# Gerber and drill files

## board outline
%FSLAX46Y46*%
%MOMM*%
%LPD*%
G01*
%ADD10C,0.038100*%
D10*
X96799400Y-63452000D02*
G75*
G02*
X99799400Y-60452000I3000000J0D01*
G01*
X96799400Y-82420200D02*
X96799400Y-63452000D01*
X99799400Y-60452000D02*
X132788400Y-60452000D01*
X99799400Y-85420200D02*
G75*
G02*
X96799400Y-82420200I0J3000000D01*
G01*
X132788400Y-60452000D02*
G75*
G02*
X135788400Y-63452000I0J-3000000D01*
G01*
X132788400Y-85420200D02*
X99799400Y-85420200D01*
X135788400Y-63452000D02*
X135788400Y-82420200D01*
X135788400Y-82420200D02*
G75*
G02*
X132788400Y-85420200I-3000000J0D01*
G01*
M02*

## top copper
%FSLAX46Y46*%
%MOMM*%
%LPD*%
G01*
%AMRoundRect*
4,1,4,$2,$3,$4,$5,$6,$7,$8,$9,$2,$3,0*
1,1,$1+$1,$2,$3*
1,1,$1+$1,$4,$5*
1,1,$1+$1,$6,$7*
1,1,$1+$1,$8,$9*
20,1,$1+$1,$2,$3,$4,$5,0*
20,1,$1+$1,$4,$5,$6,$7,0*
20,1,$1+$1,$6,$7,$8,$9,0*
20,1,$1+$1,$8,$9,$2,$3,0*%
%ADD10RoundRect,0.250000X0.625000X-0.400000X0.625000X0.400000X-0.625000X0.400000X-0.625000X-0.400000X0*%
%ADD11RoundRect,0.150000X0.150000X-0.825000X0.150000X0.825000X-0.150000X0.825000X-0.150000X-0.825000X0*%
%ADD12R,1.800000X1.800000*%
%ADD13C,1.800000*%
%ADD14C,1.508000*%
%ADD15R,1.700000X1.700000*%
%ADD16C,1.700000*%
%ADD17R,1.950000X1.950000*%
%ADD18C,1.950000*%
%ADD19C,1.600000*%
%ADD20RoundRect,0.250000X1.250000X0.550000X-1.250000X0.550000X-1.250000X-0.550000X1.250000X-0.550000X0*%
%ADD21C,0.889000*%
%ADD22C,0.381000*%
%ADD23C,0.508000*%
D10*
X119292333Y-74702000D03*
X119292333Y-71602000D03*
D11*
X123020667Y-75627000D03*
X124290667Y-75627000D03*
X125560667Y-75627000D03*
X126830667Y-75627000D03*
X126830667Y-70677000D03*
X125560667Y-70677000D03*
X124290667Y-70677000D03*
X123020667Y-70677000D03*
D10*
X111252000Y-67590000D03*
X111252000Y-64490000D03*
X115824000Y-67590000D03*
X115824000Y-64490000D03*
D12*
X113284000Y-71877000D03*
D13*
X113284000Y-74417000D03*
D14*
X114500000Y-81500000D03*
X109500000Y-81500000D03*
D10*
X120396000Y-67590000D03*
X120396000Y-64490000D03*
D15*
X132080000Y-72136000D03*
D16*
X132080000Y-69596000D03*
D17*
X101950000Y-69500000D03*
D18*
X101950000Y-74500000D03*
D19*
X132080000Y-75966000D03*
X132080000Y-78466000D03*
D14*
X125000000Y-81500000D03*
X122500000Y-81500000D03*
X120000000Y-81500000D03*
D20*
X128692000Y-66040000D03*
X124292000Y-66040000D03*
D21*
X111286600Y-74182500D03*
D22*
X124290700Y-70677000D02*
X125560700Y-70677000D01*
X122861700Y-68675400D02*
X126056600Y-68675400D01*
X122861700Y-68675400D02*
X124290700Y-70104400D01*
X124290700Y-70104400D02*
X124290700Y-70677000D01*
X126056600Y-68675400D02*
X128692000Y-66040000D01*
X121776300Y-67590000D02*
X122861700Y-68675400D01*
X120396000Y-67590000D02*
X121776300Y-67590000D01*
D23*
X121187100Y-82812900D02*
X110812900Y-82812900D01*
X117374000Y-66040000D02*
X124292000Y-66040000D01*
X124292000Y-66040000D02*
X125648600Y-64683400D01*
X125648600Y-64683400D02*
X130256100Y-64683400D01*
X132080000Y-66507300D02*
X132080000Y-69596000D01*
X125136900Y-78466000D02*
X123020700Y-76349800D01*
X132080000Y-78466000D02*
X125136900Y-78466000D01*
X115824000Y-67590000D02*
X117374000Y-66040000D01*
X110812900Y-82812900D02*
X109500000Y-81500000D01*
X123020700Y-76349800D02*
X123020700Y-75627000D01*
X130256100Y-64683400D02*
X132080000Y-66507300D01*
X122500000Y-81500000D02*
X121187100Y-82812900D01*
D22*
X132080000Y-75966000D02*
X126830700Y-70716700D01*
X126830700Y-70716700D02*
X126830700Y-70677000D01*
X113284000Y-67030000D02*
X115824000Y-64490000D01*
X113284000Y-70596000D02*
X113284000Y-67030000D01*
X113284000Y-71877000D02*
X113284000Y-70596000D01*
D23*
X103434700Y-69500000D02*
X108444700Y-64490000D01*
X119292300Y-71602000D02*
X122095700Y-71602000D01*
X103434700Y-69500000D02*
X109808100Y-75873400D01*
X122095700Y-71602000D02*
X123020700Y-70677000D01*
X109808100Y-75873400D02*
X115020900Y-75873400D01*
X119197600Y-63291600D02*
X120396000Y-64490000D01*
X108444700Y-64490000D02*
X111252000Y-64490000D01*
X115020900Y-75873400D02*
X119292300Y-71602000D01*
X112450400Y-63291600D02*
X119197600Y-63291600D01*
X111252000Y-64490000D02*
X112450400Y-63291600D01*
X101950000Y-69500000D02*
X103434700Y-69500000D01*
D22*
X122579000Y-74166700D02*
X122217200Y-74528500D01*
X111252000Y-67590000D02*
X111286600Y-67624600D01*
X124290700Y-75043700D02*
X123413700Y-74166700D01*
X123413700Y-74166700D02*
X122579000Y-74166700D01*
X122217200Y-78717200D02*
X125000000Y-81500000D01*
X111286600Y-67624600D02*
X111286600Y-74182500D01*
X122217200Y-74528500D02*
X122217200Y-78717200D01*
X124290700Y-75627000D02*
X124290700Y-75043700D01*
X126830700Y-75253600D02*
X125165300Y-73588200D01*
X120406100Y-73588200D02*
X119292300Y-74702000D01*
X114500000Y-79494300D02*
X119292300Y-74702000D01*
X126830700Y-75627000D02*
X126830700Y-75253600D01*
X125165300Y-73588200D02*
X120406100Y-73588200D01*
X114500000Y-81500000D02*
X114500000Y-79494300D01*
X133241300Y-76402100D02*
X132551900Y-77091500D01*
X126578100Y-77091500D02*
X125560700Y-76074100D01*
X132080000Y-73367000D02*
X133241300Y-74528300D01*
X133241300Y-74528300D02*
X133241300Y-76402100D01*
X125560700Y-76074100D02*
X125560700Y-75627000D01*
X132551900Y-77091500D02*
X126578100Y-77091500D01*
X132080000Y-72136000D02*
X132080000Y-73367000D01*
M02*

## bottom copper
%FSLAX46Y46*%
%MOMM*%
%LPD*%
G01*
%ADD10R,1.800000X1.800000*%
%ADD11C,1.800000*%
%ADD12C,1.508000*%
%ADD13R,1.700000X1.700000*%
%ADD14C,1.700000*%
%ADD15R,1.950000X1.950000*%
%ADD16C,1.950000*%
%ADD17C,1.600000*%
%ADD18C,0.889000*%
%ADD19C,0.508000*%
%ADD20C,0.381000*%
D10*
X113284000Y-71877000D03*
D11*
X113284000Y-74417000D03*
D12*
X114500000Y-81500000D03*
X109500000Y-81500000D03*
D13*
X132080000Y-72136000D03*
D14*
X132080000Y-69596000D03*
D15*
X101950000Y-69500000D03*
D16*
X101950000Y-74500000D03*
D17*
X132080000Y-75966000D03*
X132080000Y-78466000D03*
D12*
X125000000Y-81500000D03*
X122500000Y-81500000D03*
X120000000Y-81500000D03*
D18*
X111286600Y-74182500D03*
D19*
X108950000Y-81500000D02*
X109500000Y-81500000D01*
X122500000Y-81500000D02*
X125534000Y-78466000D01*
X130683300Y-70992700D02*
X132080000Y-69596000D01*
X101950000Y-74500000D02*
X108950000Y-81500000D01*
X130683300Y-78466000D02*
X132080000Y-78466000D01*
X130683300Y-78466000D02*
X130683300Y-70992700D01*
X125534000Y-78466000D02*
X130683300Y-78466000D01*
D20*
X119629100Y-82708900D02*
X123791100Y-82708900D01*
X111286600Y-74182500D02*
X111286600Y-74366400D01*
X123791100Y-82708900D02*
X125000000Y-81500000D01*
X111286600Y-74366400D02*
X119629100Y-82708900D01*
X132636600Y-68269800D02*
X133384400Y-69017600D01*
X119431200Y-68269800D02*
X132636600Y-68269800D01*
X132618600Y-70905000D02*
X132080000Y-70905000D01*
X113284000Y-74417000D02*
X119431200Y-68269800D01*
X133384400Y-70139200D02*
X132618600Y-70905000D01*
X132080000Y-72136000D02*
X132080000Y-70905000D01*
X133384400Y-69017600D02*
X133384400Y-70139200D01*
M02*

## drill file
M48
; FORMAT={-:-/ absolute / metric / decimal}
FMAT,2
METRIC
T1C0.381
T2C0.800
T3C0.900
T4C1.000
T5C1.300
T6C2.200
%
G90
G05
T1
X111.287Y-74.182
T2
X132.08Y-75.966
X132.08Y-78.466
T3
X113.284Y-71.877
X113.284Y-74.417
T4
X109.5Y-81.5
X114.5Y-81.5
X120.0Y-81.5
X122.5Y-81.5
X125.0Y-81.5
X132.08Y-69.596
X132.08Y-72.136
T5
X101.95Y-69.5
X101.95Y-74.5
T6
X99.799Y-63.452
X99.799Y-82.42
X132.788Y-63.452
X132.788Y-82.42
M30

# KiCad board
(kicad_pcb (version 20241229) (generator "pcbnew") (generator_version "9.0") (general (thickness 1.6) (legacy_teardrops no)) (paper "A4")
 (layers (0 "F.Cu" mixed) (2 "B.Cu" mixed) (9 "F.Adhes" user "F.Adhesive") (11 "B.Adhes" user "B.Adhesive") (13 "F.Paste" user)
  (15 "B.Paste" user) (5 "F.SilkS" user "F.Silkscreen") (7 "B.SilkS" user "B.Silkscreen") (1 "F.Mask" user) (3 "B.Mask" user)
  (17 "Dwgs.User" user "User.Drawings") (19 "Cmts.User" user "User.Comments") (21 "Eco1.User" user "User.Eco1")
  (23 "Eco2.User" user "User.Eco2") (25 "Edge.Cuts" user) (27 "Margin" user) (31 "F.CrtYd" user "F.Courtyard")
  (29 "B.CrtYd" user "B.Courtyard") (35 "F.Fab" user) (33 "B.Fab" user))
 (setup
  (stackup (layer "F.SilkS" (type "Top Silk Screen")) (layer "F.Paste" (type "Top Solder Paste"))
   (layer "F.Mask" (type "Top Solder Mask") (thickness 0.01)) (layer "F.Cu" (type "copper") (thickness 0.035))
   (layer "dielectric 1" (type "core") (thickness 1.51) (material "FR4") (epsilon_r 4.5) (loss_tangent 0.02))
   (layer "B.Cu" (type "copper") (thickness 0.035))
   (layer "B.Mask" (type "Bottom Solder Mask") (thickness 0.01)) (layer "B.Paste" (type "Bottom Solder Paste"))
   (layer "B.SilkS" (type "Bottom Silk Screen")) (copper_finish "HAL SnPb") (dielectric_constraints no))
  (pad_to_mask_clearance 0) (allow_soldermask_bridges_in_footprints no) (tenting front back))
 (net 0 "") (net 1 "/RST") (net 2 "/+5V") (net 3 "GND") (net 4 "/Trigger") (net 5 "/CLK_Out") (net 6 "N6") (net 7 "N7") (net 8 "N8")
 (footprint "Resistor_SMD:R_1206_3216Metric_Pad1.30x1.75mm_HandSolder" (layer "F.Cu") (at 119.292333 73.152 90)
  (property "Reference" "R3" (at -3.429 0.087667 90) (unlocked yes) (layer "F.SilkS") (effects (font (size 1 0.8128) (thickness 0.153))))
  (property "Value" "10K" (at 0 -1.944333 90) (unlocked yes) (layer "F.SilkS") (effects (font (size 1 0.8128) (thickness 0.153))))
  (pad "1" smd roundrect (at -1.55 0 90) (size 1.3 1.75) (layers "F.Cu" "F.Mask" "F.Paste") (roundrect_rratio 0.192308) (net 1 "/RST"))
  (pad "2" smd roundrect (at 1.55 0 90) (size 1.3 1.75) (layers "F.Cu" "F.Mask" "F.Paste") (roundrect_rratio 0.192308) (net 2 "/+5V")))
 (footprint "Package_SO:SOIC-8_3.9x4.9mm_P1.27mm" (layer "F.Cu") (at 124.925667 73.152 90)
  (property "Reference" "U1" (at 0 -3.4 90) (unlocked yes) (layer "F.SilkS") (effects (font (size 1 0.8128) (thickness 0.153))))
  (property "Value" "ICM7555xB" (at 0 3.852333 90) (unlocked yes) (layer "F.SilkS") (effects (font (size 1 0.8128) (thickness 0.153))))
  (pad "1" smd roundrect (at -2.475 -1.905 90) (size 1.95 0.6) (layers "F.Cu" "F.Mask" "F.Paste") (roundrect_rratio 0.25) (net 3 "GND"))
  (pad "2" smd roundrect (at -2.475 -0.635 90) (size 1.95 0.6) (layers "F.Cu" "F.Mask" "F.Paste") (roundrect_rratio 0.25) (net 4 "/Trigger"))
  (pad "3" smd roundrect (at -2.475 0.635 90) (size 1.95 0.6) (layers "F.Cu" "F.Mask" "F.Paste") (roundrect_rratio 0.25) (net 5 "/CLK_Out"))
  (pad "4" smd roundrect (at -2.475 1.905 90) (size 1.95 0.6) (layers "F.Cu" "F.Mask" "F.Paste") (roundrect_rratio 0.25) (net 1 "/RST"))
  (pad "5" smd roundrect (at 2.475 1.905 90) (size 1.95 0.6) (layers "F.Cu" "F.Mask" "F.Paste") (roundrect_rratio 0.25) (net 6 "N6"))
  (pad "6" smd roundrect (at 2.475 0.635 90) (size 1.95 0.6) (layers "F.Cu" "F.Mask" "F.Paste") (roundrect_rratio 0.25) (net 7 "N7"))
  (pad "7" smd roundrect (at 2.475 -0.635 90) (size 1.95 0.6) (layers "F.Cu" "F.Mask" "F.Paste") (roundrect_rratio 0.25) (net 7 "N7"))
  (pad "8" smd roundrect (at 2.475 -1.905 90) (size 1.95 0.6) (layers "F.Cu" "F.Mask" "F.Paste") (roundrect_rratio 0.25) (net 2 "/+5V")))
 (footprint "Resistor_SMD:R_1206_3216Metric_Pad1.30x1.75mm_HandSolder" (layer "F.Cu") (at 111.252 66.04 90)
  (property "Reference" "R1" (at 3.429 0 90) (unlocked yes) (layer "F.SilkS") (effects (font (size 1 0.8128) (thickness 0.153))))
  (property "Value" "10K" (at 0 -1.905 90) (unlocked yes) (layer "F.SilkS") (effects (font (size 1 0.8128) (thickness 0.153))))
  (pad "1" smd roundrect (at -1.55 0 90) (size 1.3 1.75) (layers "F.Cu" "F.Mask" "F.Paste") (roundrect_rratio 0.192308) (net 4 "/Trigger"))
  (pad "2" smd roundrect (at 1.55 0 90) (size 1.3 1.75) (layers "F.Cu" "F.Mask" "F.Paste") (roundrect_rratio 0.192308) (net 2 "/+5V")))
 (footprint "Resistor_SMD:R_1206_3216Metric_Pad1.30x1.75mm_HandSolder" (layer "F.Cu") (at 115.824 66.04 90)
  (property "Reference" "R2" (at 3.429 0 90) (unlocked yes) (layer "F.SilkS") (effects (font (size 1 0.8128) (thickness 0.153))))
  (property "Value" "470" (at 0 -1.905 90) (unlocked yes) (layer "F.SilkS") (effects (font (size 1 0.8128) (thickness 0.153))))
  (pad "1" smd roundrect (at -1.55 0 90) (size 1.3 1.75) (layers "F.Cu" "F.Mask" "F.Paste") (roundrect_rratio 0.192308) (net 3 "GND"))
  (pad "2" smd roundrect (at 1.55 0 90) (size 1.3 1.75) (layers "F.Cu" "F.Mask" "F.Paste") (roundrect_rratio 0.192308) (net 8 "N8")))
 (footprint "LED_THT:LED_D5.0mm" (layer "F.Cu") (at 113.284 71.877 -90)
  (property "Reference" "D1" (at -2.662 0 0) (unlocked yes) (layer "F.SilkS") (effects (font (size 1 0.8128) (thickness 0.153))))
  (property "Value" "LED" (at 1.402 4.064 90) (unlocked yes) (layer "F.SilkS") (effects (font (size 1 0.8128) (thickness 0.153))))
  (pad "1" thru_hole rect (at 0 0 270) (size 1.8 1.8) (drill 0.9) (layers "*.Cu" "*.Mask") (remove_unused_layers no) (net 8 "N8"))
  (pad "2" thru_hole circle (at 2.54 0 270) (size 1.8 1.8) (drill 0.9) (layers "*.Cu" "*.Mask") (remove_unused_layers no) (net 5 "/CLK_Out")))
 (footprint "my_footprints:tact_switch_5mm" (layer "F.Cu") (at 112 81.5 180)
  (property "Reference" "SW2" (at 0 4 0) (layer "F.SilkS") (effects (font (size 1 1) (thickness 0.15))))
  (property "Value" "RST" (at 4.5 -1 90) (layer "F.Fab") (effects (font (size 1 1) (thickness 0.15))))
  (pad "1" thru_hole circle (at -2.5 0 180) (size 1.508 1.508) (drill 1) (layers "*.Cu" "*.Mask") (remove_unused_layers no) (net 1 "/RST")
   (solder_mask_margin 0.102))
  (pad "2" thru_hole circle (at 2.5 0 180) (size 1.508 1.508) (drill 1) (layers "*.Cu" "*.Mask") (remove_unused_layers no) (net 3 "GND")
   (solder_mask_margin 0.102)))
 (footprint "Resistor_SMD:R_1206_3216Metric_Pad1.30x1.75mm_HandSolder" (layer "F.Cu") (at 120.396 66.04 90)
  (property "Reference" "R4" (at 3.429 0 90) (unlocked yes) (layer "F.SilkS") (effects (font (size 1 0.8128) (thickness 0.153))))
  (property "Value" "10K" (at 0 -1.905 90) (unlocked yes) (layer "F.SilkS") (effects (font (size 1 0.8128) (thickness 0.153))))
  (pad "1" smd roundrect (at -1.55 0 90) (size 1.3 1.75) (layers "F.Cu" "F.Mask" "F.Paste") (roundrect_rratio 0.192308) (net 7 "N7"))
  (pad "2" smd roundrect (at 1.55 0 90) (size 1.3 1.75) (layers "F.Cu" "F.Mask" "F.Paste") (roundrect_rratio 0.192308) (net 2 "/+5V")))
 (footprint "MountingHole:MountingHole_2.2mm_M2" (layer "F.Cu") (at 99.7994 63.452)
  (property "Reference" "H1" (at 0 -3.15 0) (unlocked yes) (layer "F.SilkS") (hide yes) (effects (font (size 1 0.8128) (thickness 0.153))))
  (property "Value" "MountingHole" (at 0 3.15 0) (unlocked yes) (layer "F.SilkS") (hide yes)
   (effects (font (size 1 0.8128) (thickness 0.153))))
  (pad "" np_thru_hole circle (at 0 0) (size 2.2 2.2) (drill 2.2) (layers "*.Cu" "*.Mask")))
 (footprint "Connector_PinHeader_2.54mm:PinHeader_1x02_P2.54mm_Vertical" (layer "F.Cu") (at 132.08 72.136 180)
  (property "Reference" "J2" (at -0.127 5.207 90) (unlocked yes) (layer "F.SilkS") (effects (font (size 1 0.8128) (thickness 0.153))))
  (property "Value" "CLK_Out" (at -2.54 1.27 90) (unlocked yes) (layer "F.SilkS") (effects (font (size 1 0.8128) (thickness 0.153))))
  (pad "1" thru_hole rect (at 0 0 180) (size 1.7 1.7) (drill 1) (layers "*.Cu" "*.Mask") (remove_unused_layers no) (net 5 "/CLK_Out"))
  (pad "2" thru_hole circle (at 0 2.54 180) (size 1.7 1.7) (drill 1) (layers "*.Cu" "*.Mask") (remove_unused_layers no) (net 3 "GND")))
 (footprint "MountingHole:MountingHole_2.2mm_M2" (layer "F.Cu") (at 132.7884 82.4202)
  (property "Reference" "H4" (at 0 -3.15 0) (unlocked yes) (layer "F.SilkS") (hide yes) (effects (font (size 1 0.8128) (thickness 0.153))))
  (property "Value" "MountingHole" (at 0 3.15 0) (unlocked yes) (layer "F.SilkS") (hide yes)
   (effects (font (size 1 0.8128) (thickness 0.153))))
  (pad "" np_thru_hole circle (at 0 0) (size 2.2 2.2) (drill 2.2) (layers "*.Cu" "*.Mask")))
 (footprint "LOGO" (layer "F.Cu") (at 105.5 63.5)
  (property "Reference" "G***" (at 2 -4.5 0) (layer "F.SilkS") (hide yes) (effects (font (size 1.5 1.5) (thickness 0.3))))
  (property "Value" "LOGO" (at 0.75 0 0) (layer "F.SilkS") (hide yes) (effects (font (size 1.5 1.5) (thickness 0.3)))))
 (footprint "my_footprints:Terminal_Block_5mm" (layer "F.Cu") (at 101.95 72 -90)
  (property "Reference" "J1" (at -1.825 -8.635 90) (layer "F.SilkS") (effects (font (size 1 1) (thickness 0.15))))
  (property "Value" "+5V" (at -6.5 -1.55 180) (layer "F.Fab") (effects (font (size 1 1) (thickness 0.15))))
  (pad "1" thru_hole rect (at -2.5 0 270) (size 1.95 1.95) (drill 1.3) (layers "*.Cu" "*.Mask") (remove_unused_layers no) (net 2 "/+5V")
   (solder_mask_margin 0.102))
  (pad "2" thru_hole circle (at 2.5 0 270) (size 1.95 1.95) (drill 1.3) (layers "*.Cu" "*.Mask") (remove_unused_layers no) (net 3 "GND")
   (solder_mask_margin 0.102)))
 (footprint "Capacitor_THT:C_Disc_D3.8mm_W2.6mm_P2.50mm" (layer "F.Cu") (at 132.08 75.966 -90)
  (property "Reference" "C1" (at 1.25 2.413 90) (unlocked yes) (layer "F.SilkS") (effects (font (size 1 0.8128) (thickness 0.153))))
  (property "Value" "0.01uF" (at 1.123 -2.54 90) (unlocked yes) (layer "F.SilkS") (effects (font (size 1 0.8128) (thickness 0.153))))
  (pad "1" thru_hole circle (at 0 0 270) (size 1.6 1.6) (drill 0.8) (layers "*.Cu" "*.Mask") (remove_unused_layers no) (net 6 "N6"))
  (pad "2" thru_hole circle (at 2.5 0 270) (size 1.6 1.6) (drill 0.8) (layers "*.Cu" "*.Mask") (remove_unused_layers no) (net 3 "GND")))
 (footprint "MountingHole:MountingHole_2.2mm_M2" (layer "F.Cu") (at 132.7884 63.452)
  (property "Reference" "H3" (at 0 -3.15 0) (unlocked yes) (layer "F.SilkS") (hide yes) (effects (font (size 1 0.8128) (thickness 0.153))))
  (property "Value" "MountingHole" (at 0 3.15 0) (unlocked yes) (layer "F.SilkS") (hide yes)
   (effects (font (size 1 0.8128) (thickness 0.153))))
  (pad "" np_thru_hole circle (at 0 0) (size 2.2 2.2) (drill 2.2) (layers "*.Cu" "*.Mask")))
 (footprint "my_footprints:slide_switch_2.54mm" (layer "F.Cu") (at 122.5 81.5 180)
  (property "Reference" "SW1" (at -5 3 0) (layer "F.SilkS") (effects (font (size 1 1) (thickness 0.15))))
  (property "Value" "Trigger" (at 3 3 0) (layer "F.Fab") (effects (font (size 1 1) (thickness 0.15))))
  (pad "1" thru_hole circle (at -2.5 0 180) (size 1.508 1.508) (drill 1) (layers "*.Cu" "*.Mask") (remove_unused_layers no)
   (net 4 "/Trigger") (solder_mask_margin 0.102))
  (pad "2" thru_hole circle (at 0 0 180) (size 1.508 1.508) (drill 1) (layers "*.Cu" "*.Mask") (remove_unused_layers no) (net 3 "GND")
   (solder_mask_margin 0.102))
  (pad "3" thru_hole circle (at 2.5 0 180) (size 1.508 1.508) (drill 1) (layers "*.Cu" "*.Mask") (remove_unused_layers no)
   (solder_mask_margin 0.102)))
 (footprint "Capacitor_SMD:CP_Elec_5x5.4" (layer "F.Cu") (at 126.492 66.04 180)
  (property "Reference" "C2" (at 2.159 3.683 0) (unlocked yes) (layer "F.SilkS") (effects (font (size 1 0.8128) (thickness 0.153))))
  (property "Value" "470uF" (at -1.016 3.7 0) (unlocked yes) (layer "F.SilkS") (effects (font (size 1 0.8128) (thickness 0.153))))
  (pad "1" smd roundrect (at -2.2 0 180) (size 3 1.6) (layers "F.Cu" "F.Mask" "F.Paste") (roundrect_rratio 0.15625) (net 7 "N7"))
  (pad "2" smd roundrect (at 2.2 0 180) (size 3 1.6) (layers "F.Cu" "F.Mask" "F.Paste") (roundrect_rratio 0.15625) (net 3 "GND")))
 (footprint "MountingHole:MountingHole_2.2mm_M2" (layer "F.Cu") (at 99.7994 82.4202)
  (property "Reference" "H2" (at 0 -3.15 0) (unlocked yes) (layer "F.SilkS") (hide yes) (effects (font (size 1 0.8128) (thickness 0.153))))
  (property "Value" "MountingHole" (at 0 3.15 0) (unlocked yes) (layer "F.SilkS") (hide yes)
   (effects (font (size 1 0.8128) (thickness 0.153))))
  (pad "" np_thru_hole circle (at 0 0) (size 2.2 2.2) (drill 2.2) (layers "*.Cu" "*.Mask")))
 (gr_arc (start 96.7994 63.452) (mid 97.67808 61.33068) (end 99.7994 60.452) (stroke (width 0.0381) (type default)) (layer "Edge.Cuts"))
 (gr_line (start 96.7994 82.4202) (end 96.7994 63.452) (stroke (width 0.0381) (type default)) (layer "Edge.Cuts"))
 (gr_line (start 99.7994 60.452) (end 132.7884 60.452) (stroke (width 0.0381) (type default)) (layer "Edge.Cuts"))
 (gr_arc (start 99.7994 85.4202) (mid 97.67808 84.54152) (end 96.7994 82.4202) (stroke (width 0.0381) (type default)) (layer "Edge.Cuts"))
 (gr_arc (start 132.7884 60.452) (mid 134.90972 61.33068) (end 135.7884 63.452) (stroke (width 0.0381) (type default)) (layer "Edge.Cuts"))
 (gr_line (start 132.7884 85.4202) (end 99.7994 85.4202) (stroke (width 0.0381) (type default)) (layer "Edge.Cuts"))
 (gr_line (start 135.7884 63.452) (end 135.7884 82.4202) (stroke (width 0.0381) (type default)) (layer "Edge.Cuts"))
 (gr_arc (start 135.7884 82.4202) (mid 134.90972 84.54152) (end 132.7884 85.4202) (stroke (width 0.0381) (type default)) (layer "Edge.Cuts"))
 (segment (start 124.290700 70.677000) (end 125.560700 70.677000) (width 0.381000) (layer "F.Cu") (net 7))
 (segment (start 122.861700 68.675400) (end 126.056600 68.675400) (width 0.381000) (layer "F.Cu") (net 7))
 (segment (start 122.861700 68.675400) (end 124.290700 70.104400) (width 0.381000) (layer "F.Cu") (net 7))
 (segment (start 124.290700 70.104400) (end 124.290700 70.677000) (width 0.381000) (layer "F.Cu") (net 7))
 (segment (start 126.056600 68.675400) (end 128.692000 66.040000) (width 0.381000) (layer "F.Cu") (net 7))
 (segment (start 121.776300 67.590000) (end 122.861700 68.675400) (width 0.381000) (layer "F.Cu") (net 7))
 (segment (start 120.396000 67.590000) (end 121.776300 67.590000) (width 0.381000) (layer "F.Cu") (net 7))
 (segment (start 121.187100 82.812900) (end 110.812900 82.812900) (width 0.508000) (layer "F.Cu") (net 3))
 (segment (start 117.374000 66.040000) (end 124.292000 66.040000) (width 0.508000) (layer "F.Cu") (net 3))
 (segment (start 124.292000 66.040000) (end 125.648600 64.683400) (width 0.508000) (layer "F.Cu") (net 3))
 (segment (start 125.648600 64.683400) (end 130.256100 64.683400) (width 0.508000) (layer "F.Cu") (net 3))
 (segment (start 132.080000 66.507300) (end 132.080000 69.596000) (width 0.508000) (layer "F.Cu") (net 3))
 (segment (start 125.136900 78.466000) (end 123.020700 76.349800) (width 0.508000) (layer "F.Cu") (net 3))
 (segment (start 132.080000 78.466000) (end 125.136900 78.466000) (width 0.508000) (layer "F.Cu") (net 3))
 (segment (start 115.824000 67.590000) (end 117.374000 66.040000) (width 0.508000) (layer "F.Cu") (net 3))
 (segment (start 110.812900 82.812900) (end 109.500000 81.500000) (width 0.508000) (layer "F.Cu") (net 3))
 (segment (start 123.020700 76.349800) (end 123.020700 75.627000) (width 0.508000) (layer "F.Cu") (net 3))
 (segment (start 130.256100 64.683400) (end 132.080000 66.507300) (width 0.508000) (layer "F.Cu") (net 3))
 (segment (start 122.500000 81.500000) (end 121.187100 82.812900) (width 0.508000) (layer "F.Cu") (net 3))
 (segment (start 108.950000 81.500000) (end 109.500000 81.500000) (width 0.508000) (layer "B.Cu") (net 3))
 (segment (start 122.500000 81.500000) (end 125.534000 78.466000) (width 0.508000) (layer "B.Cu") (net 3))
 (segment (start 130.683300 70.992700) (end 132.080000 69.596000) (width 0.508000) (layer "B.Cu") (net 3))
 (segment (start 101.950000 74.500000) (end 108.950000 81.500000) (width 0.508000) (layer "B.Cu") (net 3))
 (segment (start 130.683300 78.466000) (end 132.080000 78.466000) (width 0.508000) (layer "B.Cu") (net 3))
 (segment (start 130.683300 78.466000) (end 130.683300 70.992700) (width 0.508000) (layer "B.Cu") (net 3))
 (segment (start 125.534000 78.466000) (end 130.683300 78.466000) (width 0.508000) (layer "B.Cu") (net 3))
 (segment (start 132.080000 75.966000) (end 126.830700 70.716700) (width 0.381000) (layer "F.Cu") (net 6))
 (segment (start 126.830700 70.716700) (end 126.830700 70.677000) (width 0.381000) (layer "F.Cu") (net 6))
 (segment (start 113.284000 67.030000) (end 115.824000 64.490000) (width 0.381000) (layer "F.Cu") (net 8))
 (segment (start 113.284000 70.596000) (end 113.284000 67.030000) (width 0.381000) (layer "F.Cu") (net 8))
 (segment (start 113.284000 71.877000) (end 113.284000 70.596000) (width 0.381000) (layer "F.Cu") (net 8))
 (segment (start 103.434700 69.500000) (end 108.444700 64.490000) (width 0.508000) (layer "F.Cu") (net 2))
 (segment (start 119.292300 71.602000) (end 122.095700 71.602000) (width 0.508000) (layer "F.Cu") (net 2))
 (segment (start 103.434700 69.500000) (end 109.808100 75.873400) (width 0.508000) (layer "F.Cu") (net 2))
 (segment (start 122.095700 71.602000) (end 123.020700 70.677000) (width 0.508000) (layer "F.Cu") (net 2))
 (segment (start 109.808100 75.873400) (end 115.020900 75.873400) (width 0.508000) (layer "F.Cu") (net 2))
 (segment (start 119.197600 63.291600) (end 120.396000 64.490000) (width 0.508000) (layer "F.Cu") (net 2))
 (segment (start 108.444700 64.490000) (end 111.252000 64.490000) (width 0.508000) (layer "F.Cu") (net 2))
 (segment (start 115.020900 75.873400) (end 119.292300 71.602000) (width 0.508000) (layer "F.Cu") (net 2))
 (segment (start 112.450400 63.291600) (end 119.197600 63.291600) (width 0.508000) (layer "F.Cu") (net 2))
 (segment (start 111.252000 64.490000) (end 112.450400 63.291600) (width 0.508000) (layer "F.Cu") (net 2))
 (segment (start 101.950000 69.500000) (end 103.434700 69.500000) (width 0.508000) (layer "F.Cu") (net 2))
 (segment (start 122.579000 74.166700) (end 122.217200 74.528500) (width 0.381000) (layer "F.Cu") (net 4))
 (segment (start 111.252000 67.590000) (end 111.286600 67.624600) (width 0.381000) (layer "F.Cu") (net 4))
 (segment (start 124.290700 75.043700) (end 123.413700 74.166700) (width 0.381000) (layer "F.Cu") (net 4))
 (segment (start 123.413700 74.166700) (end 122.579000 74.166700) (width 0.381000) (layer "F.Cu") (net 4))
 (segment (start 122.217200 78.717200) (end 125.000000 81.500000) (width 0.381000) (layer "F.Cu") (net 4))
 (segment (start 111.286600 67.624600) (end 111.286600 74.182500) (width 0.381000) (layer "F.Cu") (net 4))
 (segment (start 122.217200 74.528500) (end 122.217200 78.717200) (width 0.381000) (layer "F.Cu") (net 4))
 (segment (start 124.290700 75.627000) (end 124.290700 75.043700) (width 0.381000) (layer "F.Cu") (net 4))
 (segment (start 119.629100 82.708900) (end 123.791100 82.708900) (width 0.381000) (layer "B.Cu") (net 4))
 (segment (start 111.286600 74.182500) (end 111.286600 74.366400) (width 0.381000) (layer "B.Cu") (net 4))
 (segment (start 123.791100 82.708900) (end 125.000000 81.500000) (width 0.381000) (layer "B.Cu") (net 4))
 (segment (start 111.286600 74.366400) (end 119.629100 82.708900) (width 0.381000) (layer "B.Cu") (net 4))
 (segment (start 126.830700 75.253600) (end 125.165300 73.588200) (width 0.381000) (layer "F.Cu") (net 1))
 (segment (start 120.406100 73.588200) (end 119.292300 74.702000) (width 0.381000) (layer "F.Cu") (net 1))
 (segment (start 114.500000 79.494300) (end 119.292300 74.702000) (width 0.381000) (layer "F.Cu") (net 1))
 (segment (start 126.830700 75.627000) (end 126.830700 75.253600) (width 0.381000) (layer "F.Cu") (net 1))
 (segment (start 125.165300 73.588200) (end 120.406100 73.588200) (width 0.381000) (layer "F.Cu") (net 1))
 (segment (start 114.500000 81.500000) (end 114.500000 79.494300) (width 0.381000) (layer "F.Cu") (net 1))
 (segment (start 133.241300 76.402100) (end 132.551900 77.091500) (width 0.381000) (layer "F.Cu") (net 5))
 (segment (start 126.578100 77.091500) (end 125.560700 76.074100) (width 0.381000) (layer "F.Cu") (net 5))
 (segment (start 132.080000 73.367000) (end 133.241300 74.528300) (width 0.381000) (layer "F.Cu") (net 5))
 (segment (start 133.241300 74.528300) (end 133.241300 76.402100) (width 0.381000) (layer "F.Cu") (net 5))
 (segment (start 125.560700 76.074100) (end 125.560700 75.627000) (width 0.381000) (layer "F.Cu") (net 5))
 (segment (start 132.551900 77.091500) (end 126.578100 77.091500) (width 0.381000) (layer "F.Cu") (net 5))
 (segment (start 132.080000 72.136000) (end 132.080000 73.367000) (width 0.381000) (layer "F.Cu") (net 5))
 (segment (start 132.636600 68.269800) (end 133.384400 69.017600) (width 0.381000) (layer "B.Cu") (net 5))
 (segment (start 119.431200 68.269800) (end 132.636600 68.269800) (width 0.381000) (layer "B.Cu") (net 5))
 (segment (start 132.618600 70.905000) (end 132.080000 70.905000) (width 0.381000) (layer "B.Cu") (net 5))
 (segment (start 113.284000 74.417000) (end 119.431200 68.269800) (width 0.381000) (layer "B.Cu") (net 5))
 (segment (start 133.384400 70.139200) (end 132.618600 70.905000) (width 0.381000) (layer "B.Cu") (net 5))
 (segment (start 132.080000 72.136000) (end 132.080000 70.905000) (width 0.381000) (layer "B.Cu") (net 5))
 (segment (start 133.384400 69.017600) (end 133.384400 70.139200) (width 0.381000) (layer "B.Cu") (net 5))
 (via (at 111.286600 74.182500) (size 0.889000) (drill 0.381000) (layers "F.Cu" "B.Cu") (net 4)))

